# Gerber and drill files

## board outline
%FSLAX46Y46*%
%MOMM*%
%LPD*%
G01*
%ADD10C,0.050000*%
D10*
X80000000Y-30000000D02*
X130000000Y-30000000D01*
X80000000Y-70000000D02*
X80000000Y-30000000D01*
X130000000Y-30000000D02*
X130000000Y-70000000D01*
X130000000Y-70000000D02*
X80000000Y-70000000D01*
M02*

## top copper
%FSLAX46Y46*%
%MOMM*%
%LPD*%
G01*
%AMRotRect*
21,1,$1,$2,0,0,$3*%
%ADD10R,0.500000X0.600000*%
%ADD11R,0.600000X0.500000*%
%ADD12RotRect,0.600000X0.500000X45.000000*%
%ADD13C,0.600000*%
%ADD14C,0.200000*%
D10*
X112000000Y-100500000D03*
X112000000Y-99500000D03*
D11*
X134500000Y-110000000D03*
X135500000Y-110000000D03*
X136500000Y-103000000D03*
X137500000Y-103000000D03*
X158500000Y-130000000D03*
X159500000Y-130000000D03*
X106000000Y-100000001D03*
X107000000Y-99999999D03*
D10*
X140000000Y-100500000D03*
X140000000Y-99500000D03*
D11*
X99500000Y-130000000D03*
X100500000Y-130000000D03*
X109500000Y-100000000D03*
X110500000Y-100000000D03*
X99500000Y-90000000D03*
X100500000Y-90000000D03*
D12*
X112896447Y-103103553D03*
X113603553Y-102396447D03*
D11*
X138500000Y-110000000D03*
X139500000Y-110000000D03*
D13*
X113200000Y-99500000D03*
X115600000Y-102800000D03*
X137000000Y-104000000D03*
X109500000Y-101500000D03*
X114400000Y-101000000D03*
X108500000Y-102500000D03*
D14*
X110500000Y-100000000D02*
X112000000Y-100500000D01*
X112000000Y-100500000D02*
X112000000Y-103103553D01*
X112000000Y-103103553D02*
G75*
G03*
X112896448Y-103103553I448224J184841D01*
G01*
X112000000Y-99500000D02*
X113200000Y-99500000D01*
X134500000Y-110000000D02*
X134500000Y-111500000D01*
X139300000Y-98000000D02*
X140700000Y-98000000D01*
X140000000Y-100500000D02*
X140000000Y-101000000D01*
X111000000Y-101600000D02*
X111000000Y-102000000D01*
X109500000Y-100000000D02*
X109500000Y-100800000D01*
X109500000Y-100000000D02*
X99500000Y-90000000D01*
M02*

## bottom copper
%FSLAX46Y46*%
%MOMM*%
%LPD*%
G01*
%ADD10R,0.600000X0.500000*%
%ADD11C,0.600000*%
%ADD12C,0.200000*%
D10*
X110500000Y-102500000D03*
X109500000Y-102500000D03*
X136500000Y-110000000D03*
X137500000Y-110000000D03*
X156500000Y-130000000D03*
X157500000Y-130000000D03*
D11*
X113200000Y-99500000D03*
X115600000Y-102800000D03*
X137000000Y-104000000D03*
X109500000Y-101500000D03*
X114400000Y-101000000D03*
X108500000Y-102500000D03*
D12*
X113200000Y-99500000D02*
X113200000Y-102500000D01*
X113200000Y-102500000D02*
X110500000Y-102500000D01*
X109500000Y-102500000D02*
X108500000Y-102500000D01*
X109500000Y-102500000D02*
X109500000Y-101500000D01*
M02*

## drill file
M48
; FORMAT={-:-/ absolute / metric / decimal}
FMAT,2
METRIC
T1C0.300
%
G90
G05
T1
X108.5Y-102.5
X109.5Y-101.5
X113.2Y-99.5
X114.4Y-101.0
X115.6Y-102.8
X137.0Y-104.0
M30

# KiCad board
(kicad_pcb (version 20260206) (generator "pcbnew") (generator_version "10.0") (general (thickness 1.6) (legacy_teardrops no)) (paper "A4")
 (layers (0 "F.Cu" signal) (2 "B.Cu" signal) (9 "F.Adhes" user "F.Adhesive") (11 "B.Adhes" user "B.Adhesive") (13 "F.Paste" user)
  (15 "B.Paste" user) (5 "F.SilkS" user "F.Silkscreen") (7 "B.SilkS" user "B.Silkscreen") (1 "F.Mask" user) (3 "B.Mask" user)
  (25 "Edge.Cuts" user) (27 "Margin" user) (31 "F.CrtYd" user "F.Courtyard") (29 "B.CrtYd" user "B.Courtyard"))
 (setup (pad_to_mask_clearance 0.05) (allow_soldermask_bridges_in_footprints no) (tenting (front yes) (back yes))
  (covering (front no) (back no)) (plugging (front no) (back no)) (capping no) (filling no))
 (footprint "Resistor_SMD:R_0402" (layer "F.Cu") (at 112 100 90)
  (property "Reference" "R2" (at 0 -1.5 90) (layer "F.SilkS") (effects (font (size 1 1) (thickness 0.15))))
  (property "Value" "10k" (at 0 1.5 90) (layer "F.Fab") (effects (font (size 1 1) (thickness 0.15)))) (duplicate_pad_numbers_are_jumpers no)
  (pad "1" smd rect (at -0.5 0 90) (size 0.6 0.5) (layers "F.Cu" "F.Mask" "F.Paste") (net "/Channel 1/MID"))
  (pad "2" smd rect (at 0.5 0 90) (size 0.6 0.5) (layers "F.Cu" "F.Mask" "F.Paste") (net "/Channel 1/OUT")))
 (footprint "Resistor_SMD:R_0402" (layer "F.Cu") (at 135 110)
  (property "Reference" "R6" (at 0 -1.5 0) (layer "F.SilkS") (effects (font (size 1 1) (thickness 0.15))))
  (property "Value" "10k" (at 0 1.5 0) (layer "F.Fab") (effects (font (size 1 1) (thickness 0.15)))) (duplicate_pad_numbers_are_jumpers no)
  (pad "1" smd rect (at -0.5 0) (size 0.6 0.5) (layers "F.Cu" "F.Mask" "F.Paste") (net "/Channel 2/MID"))
  (pad "2" smd rect (at 0.5 0) (size 0.6 0.5) (layers "F.Cu" "F.Mask" "F.Paste") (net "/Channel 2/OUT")))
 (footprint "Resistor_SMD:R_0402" (layer "F.Cu") (at 137 103)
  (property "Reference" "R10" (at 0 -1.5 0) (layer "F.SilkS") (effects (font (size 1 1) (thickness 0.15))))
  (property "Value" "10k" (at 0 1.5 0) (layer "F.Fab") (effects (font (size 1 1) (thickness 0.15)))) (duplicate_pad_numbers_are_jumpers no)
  (pad "1" smd rect (at -0.5 0) (size 0.6 0.5) (layers "F.Cu" "F.Mask" "F.Paste") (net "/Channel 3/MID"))
  (pad "2" smd rect (at 0.5 0) (size 0.6 0.5) (layers "F.Cu" "F.Mask" "F.Paste") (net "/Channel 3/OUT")))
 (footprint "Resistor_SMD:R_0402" (layer "F.Cu") (at 159 130)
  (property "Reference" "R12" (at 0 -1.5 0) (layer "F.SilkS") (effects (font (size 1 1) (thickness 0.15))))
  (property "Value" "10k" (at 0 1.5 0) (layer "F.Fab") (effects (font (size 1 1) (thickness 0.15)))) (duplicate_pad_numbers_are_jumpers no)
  (pad "1" smd rect (at -0.5 0) (size 0.6 0.5) (layers "F.Cu" "F.Mask" "F.Paste") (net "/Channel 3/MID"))
  (pad "2" smd rect (at 0.5 0) (size 0.6 0.5) (layers "F.Cu" "F.Mask" "F.Paste") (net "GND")))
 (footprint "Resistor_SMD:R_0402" (layer "F.Cu") (at 106.5 100)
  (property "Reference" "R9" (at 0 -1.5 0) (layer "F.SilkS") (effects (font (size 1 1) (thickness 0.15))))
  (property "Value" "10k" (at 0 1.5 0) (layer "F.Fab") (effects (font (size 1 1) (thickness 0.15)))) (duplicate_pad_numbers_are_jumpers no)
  (pad "1" smd rect (at -0.5 0.000001) (size 0.6 0.5) (layers "F.Cu" "F.Mask" "F.Paste") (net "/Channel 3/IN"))
  (pad "2" smd rect (at 0.5 -0.000001) (size 0.6 0.5) (layers "F.Cu" "F.Mask" "F.Paste") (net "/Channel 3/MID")))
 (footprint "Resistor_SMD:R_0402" (layer "F.Cu") (at 140 100 90)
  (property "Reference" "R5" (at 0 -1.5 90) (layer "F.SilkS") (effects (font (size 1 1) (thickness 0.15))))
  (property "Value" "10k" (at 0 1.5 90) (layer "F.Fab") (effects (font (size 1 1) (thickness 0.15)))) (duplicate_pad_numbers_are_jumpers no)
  (pad "1" smd rect (at -0.5 0 90) (size 0.6 0.5) (layers "F.Cu" "F.Mask" "F.Paste") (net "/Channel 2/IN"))
  (pad "2" smd rect (at 0.5 0 90) (size 0.6 0.5) (layers "F.Cu" "F.Mask" "F.Paste") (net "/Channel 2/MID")))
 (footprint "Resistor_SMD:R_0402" (layer "F.Cu") (at 100 130)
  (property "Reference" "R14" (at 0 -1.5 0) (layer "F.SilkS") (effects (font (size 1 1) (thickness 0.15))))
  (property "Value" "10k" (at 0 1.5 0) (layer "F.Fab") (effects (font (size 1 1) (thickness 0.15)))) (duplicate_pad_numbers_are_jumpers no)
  (pad "1" smd rect (at -0.5 0) (size 0.6 0.5) (layers "F.Cu" "F.Mask" "F.Paste") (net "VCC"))
  (pad "2" smd rect (at 0.5 0) (size 0.6 0.5) (layers "F.Cu" "F.Mask" "F.Paste") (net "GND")))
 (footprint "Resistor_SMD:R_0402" (layer "F.Cu") (at 110 100)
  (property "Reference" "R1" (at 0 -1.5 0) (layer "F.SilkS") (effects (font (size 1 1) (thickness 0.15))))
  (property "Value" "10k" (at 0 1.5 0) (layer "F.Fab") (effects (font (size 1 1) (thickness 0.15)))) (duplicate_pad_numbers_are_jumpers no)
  (pad "1" smd rect (at -0.5 0) (size 0.6 0.5) (layers "F.Cu" "F.Mask" "F.Paste") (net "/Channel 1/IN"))
  (pad "2" smd rect (at 0.5 0) (size 0.6 0.5) (layers "F.Cu" "F.Mask" "F.Paste") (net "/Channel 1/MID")))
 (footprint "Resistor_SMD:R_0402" (layer "F.Cu") (at 100 90)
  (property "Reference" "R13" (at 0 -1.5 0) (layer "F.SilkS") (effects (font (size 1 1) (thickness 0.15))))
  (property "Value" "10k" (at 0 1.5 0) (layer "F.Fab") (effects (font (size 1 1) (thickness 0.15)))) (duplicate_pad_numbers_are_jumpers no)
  (pad "1" smd rect (at -0.5 0) (size 0.6 0.5) (layers "F.Cu" "F.Mask" "F.Paste") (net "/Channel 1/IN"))
  (pad "2" smd rect (at 0.5 0) (size 0.6 0.5) (layers "F.Cu" "F.Mask" "F.Paste") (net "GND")))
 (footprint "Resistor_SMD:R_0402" (layer "F.Cu") (at 113.25 102.75 45)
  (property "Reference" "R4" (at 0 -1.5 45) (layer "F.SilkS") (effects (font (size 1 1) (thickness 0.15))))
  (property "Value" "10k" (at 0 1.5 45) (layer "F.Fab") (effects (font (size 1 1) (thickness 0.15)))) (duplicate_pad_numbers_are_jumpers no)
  (pad "1" smd rect (at -0.499999 0 45) (size 0.6 0.5) (layers "F.Cu" "F.Mask" "F.Paste") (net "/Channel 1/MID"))
  (pad "2" smd rect (at 0.499999 0 45) (size 0.6 0.5) (layers "F.Cu" "F.Mask" "F.Paste") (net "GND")))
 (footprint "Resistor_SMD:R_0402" (layer "F.Cu") (at 139 110)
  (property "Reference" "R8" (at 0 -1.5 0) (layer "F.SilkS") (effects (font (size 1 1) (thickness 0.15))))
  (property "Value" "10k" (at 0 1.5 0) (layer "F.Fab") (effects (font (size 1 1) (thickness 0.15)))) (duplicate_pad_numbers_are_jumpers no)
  (pad "1" smd rect (at -0.5 0) (size 0.6 0.5) (layers "F.Cu" "F.Mask" "F.Paste") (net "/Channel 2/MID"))
  (pad "2" smd rect (at 0.5 0) (size 0.6 0.5) (layers "F.Cu" "F.Mask" "F.Paste") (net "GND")))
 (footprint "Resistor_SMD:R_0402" (layer "B.Cu") (at 110 102.5 180)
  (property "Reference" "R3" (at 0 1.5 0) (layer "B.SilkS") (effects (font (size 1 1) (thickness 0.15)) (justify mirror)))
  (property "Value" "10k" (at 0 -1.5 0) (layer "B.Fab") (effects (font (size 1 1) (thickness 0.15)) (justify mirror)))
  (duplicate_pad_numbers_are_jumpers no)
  (pad "1" smd rect (at -0.5 0 180) (size 0.6 0.5) (layers "B.Cu" "B.Mask" "B.Paste") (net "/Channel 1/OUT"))
  (pad "2" smd rect (at 0.5 0 180) (size 0.6 0.5) (layers "B.Cu" "B.Mask" "B.Paste") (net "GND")))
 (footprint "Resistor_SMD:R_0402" (layer "B.Cu") (at 137 110)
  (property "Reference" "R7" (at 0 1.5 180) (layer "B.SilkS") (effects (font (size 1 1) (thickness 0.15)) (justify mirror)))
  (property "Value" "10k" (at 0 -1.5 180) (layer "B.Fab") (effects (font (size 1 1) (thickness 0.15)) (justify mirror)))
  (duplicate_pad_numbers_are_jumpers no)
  (pad "1" smd rect (at -0.5 0) (size 0.6 0.5) (layers "B.Cu" "B.Mask" "B.Paste") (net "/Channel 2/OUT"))
  (pad "2" smd rect (at 0.5 0) (size 0.6 0.5) (layers "B.Cu" "B.Mask" "B.Paste") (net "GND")))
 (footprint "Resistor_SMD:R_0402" (layer "B.Cu") (at 157 130)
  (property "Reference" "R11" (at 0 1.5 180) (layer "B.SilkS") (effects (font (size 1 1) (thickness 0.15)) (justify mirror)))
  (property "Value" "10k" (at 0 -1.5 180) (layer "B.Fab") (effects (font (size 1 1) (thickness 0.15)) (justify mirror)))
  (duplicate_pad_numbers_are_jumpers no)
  (pad "1" smd rect (at -0.5 0) (size 0.6 0.5) (layers "B.Cu" "B.Mask" "B.Paste") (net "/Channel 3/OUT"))
  (pad "2" smd rect (at 0.5 0) (size 0.6 0.5) (layers "B.Cu" "B.Mask" "B.Paste") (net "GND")))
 (gr_line (start 80 30) (end 130 30) (stroke (width 0.05) (type default)) (layer "Edge.Cuts"))
 (gr_line (start 80 70) (end 80 30) (stroke (width 0.05) (type default)) (layer "Edge.Cuts"))
 (gr_line (start 130 30) (end 130 70) (stroke (width 0.05) (type default)) (layer "Edge.Cuts"))
 (gr_line (start 130 70) (end 80 70) (stroke (width 0.05) (type default)) (layer "Edge.Cuts"))
 (segment (start 110.5 100) (end 112 100.5) (width 0.2) (locked yes) (layer "F.Cu") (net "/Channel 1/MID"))
 (segment (start 112 100.5) (end 112 103.103553) (width 0.2) (layer "F.Cu") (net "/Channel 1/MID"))
 (arc (start 112 103.103553) (mid 112.448223 103.403553) (end 112.896447 103.103553) (width 0.2) (layer "F.Cu") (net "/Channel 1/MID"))
 (segment (start 112 99.5) (end 113.2 99.5) (width 0.2) (layer "F.Cu") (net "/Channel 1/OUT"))
 (via (at 113.2 99.5) (size 0.6) (drill 0.3) (layers "F.Cu" "B.Cu") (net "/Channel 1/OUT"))
 (segment (start 113.2 99.5) (end 113.2 102.5) (width 0.2) (layer "B.Cu") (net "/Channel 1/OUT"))
 (segment (start 113.2 102.5) (end 110.5 102.5) (width 0.2) (layer "B.Cu") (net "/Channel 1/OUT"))
 (segment (start 134.5 110) (end 134.5 111.5) (width 0.2) (layer "F.Cu") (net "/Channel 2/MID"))
 (segment (start 139.3 98) (end 140.7 98) (width 0.2) (layer "F.Cu") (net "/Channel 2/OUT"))
 (via (at 115.6 102.8) (size 0.6) (drill 0.3) (layers "F.Cu" "B.Cu") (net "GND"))
 (via (at 137 104) (size 0.6) (drill 0.3) (layers "F.Cu" "B.Cu") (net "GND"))
 (via (at 109.5 101.5) (size 0.6) (drill 0.3) (layers "F.Cu" "B.Cu") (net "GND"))
 (via (at 114.4 101) (size 0.6) (drill 0.3) (layers "F.Cu" "B.Cu") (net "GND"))
 (via (at 108.5 102.5) (size 0.6) (drill 0.3) (layers "F.Cu" "B.Cu") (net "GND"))
 (segment (start 109.5 102.5) (end 108.5 102.5) (width 0.2) (layer "B.Cu") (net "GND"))
 (segment (start 109.5 102.5) (end 109.5 101.5) (width 0.2) (layer "B.Cu") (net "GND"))
 (segment (start 140 100.5) (end 140 101) (width 0.2) (layer "F.Cu") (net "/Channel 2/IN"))
 (segment (start 111 101.6) (end 111 102) (width 0.2) (layer "F.Cu") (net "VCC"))
 (segment (start 109.5 100) (end 109.5 100.8) (width 0.2) (layer "F.Cu") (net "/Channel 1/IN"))
 (segment (start 109.5 100) (end 99.5 90) (width 0.2) (layer "F.Cu") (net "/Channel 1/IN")))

